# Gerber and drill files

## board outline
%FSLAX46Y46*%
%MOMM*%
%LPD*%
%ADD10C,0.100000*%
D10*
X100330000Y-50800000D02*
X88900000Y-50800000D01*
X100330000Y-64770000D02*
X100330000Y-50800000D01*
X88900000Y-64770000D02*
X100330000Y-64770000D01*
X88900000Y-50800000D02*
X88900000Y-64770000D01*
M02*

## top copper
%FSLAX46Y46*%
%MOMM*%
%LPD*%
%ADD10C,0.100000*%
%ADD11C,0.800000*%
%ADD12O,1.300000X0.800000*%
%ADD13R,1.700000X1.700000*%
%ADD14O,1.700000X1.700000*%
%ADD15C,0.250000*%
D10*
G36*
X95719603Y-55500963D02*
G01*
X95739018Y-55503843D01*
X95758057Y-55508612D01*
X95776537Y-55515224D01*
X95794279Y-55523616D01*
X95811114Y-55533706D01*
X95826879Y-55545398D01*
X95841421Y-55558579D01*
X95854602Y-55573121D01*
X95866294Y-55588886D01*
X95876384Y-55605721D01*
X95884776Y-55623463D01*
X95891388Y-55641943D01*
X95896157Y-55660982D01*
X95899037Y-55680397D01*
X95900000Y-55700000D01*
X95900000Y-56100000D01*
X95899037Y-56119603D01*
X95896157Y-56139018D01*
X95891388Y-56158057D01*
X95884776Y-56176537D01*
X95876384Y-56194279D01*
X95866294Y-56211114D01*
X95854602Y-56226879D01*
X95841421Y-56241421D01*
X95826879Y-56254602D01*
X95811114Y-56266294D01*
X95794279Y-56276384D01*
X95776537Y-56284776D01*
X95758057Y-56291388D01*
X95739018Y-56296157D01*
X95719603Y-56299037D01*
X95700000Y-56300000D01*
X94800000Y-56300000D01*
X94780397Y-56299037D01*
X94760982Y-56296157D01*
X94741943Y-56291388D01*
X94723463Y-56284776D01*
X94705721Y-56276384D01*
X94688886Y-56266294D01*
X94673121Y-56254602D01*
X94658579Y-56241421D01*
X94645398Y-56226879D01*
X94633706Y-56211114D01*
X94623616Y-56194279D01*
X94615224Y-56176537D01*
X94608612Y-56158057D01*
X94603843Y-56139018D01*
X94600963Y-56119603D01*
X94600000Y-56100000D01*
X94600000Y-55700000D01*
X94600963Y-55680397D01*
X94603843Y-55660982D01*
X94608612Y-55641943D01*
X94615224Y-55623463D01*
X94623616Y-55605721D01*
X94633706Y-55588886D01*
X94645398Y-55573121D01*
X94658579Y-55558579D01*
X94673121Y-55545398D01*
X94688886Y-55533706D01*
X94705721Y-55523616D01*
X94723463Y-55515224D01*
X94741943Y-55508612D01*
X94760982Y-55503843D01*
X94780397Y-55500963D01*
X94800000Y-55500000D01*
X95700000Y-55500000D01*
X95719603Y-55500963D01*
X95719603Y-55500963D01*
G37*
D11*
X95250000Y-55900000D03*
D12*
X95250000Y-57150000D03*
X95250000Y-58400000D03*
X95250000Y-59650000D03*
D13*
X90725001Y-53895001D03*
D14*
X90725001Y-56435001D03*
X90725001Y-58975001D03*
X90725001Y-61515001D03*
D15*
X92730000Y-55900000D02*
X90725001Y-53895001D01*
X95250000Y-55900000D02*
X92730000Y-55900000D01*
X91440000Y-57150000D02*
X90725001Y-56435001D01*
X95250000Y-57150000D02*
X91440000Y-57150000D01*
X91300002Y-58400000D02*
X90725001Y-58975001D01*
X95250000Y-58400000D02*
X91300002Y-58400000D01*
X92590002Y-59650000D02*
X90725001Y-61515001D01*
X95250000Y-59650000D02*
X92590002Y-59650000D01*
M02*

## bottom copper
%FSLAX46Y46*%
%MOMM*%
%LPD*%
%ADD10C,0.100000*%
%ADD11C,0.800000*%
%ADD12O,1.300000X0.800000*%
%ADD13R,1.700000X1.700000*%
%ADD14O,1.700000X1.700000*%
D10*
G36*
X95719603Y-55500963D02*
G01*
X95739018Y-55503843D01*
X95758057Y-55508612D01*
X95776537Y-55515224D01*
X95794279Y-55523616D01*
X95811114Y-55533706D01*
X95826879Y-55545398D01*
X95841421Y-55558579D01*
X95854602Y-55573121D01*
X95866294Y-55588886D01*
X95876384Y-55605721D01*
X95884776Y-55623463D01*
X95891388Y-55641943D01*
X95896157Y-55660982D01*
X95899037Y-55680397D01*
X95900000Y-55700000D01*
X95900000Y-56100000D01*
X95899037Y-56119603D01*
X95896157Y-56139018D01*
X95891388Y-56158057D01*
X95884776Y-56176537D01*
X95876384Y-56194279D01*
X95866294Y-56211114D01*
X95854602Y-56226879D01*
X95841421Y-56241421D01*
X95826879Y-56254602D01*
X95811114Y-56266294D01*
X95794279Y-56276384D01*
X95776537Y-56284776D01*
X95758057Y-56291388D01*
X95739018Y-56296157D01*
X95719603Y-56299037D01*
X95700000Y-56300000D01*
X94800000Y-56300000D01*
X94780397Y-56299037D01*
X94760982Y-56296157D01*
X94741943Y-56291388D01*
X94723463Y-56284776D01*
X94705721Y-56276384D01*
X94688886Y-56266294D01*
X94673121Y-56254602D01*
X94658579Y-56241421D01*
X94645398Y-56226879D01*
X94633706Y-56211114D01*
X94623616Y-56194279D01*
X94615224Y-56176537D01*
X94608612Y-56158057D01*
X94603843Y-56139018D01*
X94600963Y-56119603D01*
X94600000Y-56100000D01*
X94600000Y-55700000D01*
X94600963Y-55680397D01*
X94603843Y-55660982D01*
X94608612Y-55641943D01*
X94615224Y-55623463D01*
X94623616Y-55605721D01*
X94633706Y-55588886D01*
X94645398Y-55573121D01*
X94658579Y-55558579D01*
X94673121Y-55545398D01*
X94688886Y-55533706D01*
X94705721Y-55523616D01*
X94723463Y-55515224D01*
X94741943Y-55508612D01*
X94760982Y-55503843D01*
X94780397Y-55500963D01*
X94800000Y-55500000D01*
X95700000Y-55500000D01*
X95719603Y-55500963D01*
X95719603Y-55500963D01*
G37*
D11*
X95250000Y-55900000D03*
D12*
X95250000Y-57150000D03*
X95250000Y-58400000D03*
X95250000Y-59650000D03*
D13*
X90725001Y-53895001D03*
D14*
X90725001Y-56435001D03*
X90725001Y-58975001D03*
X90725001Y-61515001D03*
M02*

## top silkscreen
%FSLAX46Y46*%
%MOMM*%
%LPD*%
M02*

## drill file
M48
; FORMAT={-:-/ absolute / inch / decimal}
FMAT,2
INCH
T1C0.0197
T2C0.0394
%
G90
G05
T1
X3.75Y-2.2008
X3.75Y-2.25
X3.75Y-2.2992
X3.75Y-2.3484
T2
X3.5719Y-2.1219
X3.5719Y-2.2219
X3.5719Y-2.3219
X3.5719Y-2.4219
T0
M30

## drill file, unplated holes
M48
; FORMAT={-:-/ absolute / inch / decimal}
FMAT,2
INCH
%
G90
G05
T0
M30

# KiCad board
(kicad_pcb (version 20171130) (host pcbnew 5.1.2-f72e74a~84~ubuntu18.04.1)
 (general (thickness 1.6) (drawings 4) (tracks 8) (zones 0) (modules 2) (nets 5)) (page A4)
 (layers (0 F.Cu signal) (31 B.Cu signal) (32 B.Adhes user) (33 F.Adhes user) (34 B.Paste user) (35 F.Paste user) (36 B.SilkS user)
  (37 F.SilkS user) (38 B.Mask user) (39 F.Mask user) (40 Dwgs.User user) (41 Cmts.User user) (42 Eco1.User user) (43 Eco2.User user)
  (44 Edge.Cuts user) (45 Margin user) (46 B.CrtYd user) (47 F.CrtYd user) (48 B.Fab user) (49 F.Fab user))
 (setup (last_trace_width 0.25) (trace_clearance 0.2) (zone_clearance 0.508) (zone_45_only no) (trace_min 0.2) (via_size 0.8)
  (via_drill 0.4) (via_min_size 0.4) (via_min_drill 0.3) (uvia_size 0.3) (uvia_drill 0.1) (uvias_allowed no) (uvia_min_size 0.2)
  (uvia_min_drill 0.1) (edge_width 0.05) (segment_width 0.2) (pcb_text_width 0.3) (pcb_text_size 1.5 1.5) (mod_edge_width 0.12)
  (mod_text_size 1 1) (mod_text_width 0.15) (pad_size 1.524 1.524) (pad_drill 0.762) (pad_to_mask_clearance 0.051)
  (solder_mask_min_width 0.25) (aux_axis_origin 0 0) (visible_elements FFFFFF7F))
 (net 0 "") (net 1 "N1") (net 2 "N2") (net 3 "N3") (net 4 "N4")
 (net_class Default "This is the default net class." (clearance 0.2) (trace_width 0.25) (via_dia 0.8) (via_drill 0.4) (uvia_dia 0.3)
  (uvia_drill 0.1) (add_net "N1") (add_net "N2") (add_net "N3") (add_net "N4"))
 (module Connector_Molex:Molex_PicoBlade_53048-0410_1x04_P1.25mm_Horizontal (layer B.Cu) (at 95.25 55.9 270)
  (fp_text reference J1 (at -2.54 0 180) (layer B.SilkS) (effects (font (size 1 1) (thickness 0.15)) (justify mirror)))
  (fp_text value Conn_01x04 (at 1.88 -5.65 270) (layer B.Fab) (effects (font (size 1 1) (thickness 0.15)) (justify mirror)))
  (pad 1 thru_hole roundrect (at 0 0 270) (size 0.8 1.3) (drill 0.5) (layers *.Cu *.Mask) (roundrect_rratio 0.25) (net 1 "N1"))
  (pad 2 thru_hole oval (at 1.25 0 270) (size 0.8 1.3) (drill 0.5) (layers *.Cu *.Mask) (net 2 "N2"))
  (pad 3 thru_hole oval (at 2.5 0 270) (size 0.8 1.3) (drill 0.5) (layers *.Cu *.Mask) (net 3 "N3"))
  (pad 4 thru_hole oval (at 3.75 0 270) (size 0.8 1.3) (drill 0.5) (layers *.Cu *.Mask) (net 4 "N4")))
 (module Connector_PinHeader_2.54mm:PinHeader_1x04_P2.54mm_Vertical (layer B.Cu) (at 90.725001 53.895001 180)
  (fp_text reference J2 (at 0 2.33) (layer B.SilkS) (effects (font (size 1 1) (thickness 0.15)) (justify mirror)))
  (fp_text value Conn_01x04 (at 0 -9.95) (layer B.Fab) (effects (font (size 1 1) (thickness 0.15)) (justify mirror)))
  (pad 1 thru_hole rect (at 0 0 180) (size 1.7 1.7) (drill 1) (layers *.Cu *.Mask) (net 1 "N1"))
  (pad 2 thru_hole oval (at 0 -2.54 180) (size 1.7 1.7) (drill 1) (layers *.Cu *.Mask) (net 2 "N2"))
  (pad 3 thru_hole oval (at 0 -5.08 180) (size 1.7 1.7) (drill 1) (layers *.Cu *.Mask) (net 3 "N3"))
  (pad 4 thru_hole oval (at 0 -7.62 180) (size 1.7 1.7) (drill 1) (layers *.Cu *.Mask) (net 4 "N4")))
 (gr_line (start 100.33 50.8) (end 88.9 50.8) (layer Edge.Cuts) (width 0.1))
 (gr_line (start 100.33 64.77) (end 100.33 50.8) (layer Edge.Cuts) (width 0.1))
 (gr_line (start 88.9 64.77) (end 100.33 64.77) (layer Edge.Cuts) (width 0.1))
 (gr_line (start 88.9 50.8) (end 88.9 64.77) (layer Edge.Cuts) (width 0.1))
 (segment (start 92.73 55.9) (end 90.725001 53.895001) (width 0.25) (layer F.Cu) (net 1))
 (segment (start 95.25 55.9) (end 92.73 55.9) (width 0.25) (layer F.Cu) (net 1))
 (segment (start 91.44 57.15) (end 90.725001 56.435001) (width 0.25) (layer F.Cu) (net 2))
 (segment (start 95.25 57.15) (end 91.44 57.15) (width 0.25) (layer F.Cu) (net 2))
 (segment (start 91.300002 58.4) (end 90.725001 58.975001) (width 0.25) (layer F.Cu) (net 3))
 (segment (start 95.25 58.4) (end 91.300002 58.4) (width 0.25) (layer F.Cu) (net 3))
 (segment (start 92.590002 59.65) (end 90.725001 61.515001) (width 0.25) (layer F.Cu) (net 4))
 (segment (start 95.25 59.65) (end 92.590002 59.65) (width 0.25) (layer F.Cu) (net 4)))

